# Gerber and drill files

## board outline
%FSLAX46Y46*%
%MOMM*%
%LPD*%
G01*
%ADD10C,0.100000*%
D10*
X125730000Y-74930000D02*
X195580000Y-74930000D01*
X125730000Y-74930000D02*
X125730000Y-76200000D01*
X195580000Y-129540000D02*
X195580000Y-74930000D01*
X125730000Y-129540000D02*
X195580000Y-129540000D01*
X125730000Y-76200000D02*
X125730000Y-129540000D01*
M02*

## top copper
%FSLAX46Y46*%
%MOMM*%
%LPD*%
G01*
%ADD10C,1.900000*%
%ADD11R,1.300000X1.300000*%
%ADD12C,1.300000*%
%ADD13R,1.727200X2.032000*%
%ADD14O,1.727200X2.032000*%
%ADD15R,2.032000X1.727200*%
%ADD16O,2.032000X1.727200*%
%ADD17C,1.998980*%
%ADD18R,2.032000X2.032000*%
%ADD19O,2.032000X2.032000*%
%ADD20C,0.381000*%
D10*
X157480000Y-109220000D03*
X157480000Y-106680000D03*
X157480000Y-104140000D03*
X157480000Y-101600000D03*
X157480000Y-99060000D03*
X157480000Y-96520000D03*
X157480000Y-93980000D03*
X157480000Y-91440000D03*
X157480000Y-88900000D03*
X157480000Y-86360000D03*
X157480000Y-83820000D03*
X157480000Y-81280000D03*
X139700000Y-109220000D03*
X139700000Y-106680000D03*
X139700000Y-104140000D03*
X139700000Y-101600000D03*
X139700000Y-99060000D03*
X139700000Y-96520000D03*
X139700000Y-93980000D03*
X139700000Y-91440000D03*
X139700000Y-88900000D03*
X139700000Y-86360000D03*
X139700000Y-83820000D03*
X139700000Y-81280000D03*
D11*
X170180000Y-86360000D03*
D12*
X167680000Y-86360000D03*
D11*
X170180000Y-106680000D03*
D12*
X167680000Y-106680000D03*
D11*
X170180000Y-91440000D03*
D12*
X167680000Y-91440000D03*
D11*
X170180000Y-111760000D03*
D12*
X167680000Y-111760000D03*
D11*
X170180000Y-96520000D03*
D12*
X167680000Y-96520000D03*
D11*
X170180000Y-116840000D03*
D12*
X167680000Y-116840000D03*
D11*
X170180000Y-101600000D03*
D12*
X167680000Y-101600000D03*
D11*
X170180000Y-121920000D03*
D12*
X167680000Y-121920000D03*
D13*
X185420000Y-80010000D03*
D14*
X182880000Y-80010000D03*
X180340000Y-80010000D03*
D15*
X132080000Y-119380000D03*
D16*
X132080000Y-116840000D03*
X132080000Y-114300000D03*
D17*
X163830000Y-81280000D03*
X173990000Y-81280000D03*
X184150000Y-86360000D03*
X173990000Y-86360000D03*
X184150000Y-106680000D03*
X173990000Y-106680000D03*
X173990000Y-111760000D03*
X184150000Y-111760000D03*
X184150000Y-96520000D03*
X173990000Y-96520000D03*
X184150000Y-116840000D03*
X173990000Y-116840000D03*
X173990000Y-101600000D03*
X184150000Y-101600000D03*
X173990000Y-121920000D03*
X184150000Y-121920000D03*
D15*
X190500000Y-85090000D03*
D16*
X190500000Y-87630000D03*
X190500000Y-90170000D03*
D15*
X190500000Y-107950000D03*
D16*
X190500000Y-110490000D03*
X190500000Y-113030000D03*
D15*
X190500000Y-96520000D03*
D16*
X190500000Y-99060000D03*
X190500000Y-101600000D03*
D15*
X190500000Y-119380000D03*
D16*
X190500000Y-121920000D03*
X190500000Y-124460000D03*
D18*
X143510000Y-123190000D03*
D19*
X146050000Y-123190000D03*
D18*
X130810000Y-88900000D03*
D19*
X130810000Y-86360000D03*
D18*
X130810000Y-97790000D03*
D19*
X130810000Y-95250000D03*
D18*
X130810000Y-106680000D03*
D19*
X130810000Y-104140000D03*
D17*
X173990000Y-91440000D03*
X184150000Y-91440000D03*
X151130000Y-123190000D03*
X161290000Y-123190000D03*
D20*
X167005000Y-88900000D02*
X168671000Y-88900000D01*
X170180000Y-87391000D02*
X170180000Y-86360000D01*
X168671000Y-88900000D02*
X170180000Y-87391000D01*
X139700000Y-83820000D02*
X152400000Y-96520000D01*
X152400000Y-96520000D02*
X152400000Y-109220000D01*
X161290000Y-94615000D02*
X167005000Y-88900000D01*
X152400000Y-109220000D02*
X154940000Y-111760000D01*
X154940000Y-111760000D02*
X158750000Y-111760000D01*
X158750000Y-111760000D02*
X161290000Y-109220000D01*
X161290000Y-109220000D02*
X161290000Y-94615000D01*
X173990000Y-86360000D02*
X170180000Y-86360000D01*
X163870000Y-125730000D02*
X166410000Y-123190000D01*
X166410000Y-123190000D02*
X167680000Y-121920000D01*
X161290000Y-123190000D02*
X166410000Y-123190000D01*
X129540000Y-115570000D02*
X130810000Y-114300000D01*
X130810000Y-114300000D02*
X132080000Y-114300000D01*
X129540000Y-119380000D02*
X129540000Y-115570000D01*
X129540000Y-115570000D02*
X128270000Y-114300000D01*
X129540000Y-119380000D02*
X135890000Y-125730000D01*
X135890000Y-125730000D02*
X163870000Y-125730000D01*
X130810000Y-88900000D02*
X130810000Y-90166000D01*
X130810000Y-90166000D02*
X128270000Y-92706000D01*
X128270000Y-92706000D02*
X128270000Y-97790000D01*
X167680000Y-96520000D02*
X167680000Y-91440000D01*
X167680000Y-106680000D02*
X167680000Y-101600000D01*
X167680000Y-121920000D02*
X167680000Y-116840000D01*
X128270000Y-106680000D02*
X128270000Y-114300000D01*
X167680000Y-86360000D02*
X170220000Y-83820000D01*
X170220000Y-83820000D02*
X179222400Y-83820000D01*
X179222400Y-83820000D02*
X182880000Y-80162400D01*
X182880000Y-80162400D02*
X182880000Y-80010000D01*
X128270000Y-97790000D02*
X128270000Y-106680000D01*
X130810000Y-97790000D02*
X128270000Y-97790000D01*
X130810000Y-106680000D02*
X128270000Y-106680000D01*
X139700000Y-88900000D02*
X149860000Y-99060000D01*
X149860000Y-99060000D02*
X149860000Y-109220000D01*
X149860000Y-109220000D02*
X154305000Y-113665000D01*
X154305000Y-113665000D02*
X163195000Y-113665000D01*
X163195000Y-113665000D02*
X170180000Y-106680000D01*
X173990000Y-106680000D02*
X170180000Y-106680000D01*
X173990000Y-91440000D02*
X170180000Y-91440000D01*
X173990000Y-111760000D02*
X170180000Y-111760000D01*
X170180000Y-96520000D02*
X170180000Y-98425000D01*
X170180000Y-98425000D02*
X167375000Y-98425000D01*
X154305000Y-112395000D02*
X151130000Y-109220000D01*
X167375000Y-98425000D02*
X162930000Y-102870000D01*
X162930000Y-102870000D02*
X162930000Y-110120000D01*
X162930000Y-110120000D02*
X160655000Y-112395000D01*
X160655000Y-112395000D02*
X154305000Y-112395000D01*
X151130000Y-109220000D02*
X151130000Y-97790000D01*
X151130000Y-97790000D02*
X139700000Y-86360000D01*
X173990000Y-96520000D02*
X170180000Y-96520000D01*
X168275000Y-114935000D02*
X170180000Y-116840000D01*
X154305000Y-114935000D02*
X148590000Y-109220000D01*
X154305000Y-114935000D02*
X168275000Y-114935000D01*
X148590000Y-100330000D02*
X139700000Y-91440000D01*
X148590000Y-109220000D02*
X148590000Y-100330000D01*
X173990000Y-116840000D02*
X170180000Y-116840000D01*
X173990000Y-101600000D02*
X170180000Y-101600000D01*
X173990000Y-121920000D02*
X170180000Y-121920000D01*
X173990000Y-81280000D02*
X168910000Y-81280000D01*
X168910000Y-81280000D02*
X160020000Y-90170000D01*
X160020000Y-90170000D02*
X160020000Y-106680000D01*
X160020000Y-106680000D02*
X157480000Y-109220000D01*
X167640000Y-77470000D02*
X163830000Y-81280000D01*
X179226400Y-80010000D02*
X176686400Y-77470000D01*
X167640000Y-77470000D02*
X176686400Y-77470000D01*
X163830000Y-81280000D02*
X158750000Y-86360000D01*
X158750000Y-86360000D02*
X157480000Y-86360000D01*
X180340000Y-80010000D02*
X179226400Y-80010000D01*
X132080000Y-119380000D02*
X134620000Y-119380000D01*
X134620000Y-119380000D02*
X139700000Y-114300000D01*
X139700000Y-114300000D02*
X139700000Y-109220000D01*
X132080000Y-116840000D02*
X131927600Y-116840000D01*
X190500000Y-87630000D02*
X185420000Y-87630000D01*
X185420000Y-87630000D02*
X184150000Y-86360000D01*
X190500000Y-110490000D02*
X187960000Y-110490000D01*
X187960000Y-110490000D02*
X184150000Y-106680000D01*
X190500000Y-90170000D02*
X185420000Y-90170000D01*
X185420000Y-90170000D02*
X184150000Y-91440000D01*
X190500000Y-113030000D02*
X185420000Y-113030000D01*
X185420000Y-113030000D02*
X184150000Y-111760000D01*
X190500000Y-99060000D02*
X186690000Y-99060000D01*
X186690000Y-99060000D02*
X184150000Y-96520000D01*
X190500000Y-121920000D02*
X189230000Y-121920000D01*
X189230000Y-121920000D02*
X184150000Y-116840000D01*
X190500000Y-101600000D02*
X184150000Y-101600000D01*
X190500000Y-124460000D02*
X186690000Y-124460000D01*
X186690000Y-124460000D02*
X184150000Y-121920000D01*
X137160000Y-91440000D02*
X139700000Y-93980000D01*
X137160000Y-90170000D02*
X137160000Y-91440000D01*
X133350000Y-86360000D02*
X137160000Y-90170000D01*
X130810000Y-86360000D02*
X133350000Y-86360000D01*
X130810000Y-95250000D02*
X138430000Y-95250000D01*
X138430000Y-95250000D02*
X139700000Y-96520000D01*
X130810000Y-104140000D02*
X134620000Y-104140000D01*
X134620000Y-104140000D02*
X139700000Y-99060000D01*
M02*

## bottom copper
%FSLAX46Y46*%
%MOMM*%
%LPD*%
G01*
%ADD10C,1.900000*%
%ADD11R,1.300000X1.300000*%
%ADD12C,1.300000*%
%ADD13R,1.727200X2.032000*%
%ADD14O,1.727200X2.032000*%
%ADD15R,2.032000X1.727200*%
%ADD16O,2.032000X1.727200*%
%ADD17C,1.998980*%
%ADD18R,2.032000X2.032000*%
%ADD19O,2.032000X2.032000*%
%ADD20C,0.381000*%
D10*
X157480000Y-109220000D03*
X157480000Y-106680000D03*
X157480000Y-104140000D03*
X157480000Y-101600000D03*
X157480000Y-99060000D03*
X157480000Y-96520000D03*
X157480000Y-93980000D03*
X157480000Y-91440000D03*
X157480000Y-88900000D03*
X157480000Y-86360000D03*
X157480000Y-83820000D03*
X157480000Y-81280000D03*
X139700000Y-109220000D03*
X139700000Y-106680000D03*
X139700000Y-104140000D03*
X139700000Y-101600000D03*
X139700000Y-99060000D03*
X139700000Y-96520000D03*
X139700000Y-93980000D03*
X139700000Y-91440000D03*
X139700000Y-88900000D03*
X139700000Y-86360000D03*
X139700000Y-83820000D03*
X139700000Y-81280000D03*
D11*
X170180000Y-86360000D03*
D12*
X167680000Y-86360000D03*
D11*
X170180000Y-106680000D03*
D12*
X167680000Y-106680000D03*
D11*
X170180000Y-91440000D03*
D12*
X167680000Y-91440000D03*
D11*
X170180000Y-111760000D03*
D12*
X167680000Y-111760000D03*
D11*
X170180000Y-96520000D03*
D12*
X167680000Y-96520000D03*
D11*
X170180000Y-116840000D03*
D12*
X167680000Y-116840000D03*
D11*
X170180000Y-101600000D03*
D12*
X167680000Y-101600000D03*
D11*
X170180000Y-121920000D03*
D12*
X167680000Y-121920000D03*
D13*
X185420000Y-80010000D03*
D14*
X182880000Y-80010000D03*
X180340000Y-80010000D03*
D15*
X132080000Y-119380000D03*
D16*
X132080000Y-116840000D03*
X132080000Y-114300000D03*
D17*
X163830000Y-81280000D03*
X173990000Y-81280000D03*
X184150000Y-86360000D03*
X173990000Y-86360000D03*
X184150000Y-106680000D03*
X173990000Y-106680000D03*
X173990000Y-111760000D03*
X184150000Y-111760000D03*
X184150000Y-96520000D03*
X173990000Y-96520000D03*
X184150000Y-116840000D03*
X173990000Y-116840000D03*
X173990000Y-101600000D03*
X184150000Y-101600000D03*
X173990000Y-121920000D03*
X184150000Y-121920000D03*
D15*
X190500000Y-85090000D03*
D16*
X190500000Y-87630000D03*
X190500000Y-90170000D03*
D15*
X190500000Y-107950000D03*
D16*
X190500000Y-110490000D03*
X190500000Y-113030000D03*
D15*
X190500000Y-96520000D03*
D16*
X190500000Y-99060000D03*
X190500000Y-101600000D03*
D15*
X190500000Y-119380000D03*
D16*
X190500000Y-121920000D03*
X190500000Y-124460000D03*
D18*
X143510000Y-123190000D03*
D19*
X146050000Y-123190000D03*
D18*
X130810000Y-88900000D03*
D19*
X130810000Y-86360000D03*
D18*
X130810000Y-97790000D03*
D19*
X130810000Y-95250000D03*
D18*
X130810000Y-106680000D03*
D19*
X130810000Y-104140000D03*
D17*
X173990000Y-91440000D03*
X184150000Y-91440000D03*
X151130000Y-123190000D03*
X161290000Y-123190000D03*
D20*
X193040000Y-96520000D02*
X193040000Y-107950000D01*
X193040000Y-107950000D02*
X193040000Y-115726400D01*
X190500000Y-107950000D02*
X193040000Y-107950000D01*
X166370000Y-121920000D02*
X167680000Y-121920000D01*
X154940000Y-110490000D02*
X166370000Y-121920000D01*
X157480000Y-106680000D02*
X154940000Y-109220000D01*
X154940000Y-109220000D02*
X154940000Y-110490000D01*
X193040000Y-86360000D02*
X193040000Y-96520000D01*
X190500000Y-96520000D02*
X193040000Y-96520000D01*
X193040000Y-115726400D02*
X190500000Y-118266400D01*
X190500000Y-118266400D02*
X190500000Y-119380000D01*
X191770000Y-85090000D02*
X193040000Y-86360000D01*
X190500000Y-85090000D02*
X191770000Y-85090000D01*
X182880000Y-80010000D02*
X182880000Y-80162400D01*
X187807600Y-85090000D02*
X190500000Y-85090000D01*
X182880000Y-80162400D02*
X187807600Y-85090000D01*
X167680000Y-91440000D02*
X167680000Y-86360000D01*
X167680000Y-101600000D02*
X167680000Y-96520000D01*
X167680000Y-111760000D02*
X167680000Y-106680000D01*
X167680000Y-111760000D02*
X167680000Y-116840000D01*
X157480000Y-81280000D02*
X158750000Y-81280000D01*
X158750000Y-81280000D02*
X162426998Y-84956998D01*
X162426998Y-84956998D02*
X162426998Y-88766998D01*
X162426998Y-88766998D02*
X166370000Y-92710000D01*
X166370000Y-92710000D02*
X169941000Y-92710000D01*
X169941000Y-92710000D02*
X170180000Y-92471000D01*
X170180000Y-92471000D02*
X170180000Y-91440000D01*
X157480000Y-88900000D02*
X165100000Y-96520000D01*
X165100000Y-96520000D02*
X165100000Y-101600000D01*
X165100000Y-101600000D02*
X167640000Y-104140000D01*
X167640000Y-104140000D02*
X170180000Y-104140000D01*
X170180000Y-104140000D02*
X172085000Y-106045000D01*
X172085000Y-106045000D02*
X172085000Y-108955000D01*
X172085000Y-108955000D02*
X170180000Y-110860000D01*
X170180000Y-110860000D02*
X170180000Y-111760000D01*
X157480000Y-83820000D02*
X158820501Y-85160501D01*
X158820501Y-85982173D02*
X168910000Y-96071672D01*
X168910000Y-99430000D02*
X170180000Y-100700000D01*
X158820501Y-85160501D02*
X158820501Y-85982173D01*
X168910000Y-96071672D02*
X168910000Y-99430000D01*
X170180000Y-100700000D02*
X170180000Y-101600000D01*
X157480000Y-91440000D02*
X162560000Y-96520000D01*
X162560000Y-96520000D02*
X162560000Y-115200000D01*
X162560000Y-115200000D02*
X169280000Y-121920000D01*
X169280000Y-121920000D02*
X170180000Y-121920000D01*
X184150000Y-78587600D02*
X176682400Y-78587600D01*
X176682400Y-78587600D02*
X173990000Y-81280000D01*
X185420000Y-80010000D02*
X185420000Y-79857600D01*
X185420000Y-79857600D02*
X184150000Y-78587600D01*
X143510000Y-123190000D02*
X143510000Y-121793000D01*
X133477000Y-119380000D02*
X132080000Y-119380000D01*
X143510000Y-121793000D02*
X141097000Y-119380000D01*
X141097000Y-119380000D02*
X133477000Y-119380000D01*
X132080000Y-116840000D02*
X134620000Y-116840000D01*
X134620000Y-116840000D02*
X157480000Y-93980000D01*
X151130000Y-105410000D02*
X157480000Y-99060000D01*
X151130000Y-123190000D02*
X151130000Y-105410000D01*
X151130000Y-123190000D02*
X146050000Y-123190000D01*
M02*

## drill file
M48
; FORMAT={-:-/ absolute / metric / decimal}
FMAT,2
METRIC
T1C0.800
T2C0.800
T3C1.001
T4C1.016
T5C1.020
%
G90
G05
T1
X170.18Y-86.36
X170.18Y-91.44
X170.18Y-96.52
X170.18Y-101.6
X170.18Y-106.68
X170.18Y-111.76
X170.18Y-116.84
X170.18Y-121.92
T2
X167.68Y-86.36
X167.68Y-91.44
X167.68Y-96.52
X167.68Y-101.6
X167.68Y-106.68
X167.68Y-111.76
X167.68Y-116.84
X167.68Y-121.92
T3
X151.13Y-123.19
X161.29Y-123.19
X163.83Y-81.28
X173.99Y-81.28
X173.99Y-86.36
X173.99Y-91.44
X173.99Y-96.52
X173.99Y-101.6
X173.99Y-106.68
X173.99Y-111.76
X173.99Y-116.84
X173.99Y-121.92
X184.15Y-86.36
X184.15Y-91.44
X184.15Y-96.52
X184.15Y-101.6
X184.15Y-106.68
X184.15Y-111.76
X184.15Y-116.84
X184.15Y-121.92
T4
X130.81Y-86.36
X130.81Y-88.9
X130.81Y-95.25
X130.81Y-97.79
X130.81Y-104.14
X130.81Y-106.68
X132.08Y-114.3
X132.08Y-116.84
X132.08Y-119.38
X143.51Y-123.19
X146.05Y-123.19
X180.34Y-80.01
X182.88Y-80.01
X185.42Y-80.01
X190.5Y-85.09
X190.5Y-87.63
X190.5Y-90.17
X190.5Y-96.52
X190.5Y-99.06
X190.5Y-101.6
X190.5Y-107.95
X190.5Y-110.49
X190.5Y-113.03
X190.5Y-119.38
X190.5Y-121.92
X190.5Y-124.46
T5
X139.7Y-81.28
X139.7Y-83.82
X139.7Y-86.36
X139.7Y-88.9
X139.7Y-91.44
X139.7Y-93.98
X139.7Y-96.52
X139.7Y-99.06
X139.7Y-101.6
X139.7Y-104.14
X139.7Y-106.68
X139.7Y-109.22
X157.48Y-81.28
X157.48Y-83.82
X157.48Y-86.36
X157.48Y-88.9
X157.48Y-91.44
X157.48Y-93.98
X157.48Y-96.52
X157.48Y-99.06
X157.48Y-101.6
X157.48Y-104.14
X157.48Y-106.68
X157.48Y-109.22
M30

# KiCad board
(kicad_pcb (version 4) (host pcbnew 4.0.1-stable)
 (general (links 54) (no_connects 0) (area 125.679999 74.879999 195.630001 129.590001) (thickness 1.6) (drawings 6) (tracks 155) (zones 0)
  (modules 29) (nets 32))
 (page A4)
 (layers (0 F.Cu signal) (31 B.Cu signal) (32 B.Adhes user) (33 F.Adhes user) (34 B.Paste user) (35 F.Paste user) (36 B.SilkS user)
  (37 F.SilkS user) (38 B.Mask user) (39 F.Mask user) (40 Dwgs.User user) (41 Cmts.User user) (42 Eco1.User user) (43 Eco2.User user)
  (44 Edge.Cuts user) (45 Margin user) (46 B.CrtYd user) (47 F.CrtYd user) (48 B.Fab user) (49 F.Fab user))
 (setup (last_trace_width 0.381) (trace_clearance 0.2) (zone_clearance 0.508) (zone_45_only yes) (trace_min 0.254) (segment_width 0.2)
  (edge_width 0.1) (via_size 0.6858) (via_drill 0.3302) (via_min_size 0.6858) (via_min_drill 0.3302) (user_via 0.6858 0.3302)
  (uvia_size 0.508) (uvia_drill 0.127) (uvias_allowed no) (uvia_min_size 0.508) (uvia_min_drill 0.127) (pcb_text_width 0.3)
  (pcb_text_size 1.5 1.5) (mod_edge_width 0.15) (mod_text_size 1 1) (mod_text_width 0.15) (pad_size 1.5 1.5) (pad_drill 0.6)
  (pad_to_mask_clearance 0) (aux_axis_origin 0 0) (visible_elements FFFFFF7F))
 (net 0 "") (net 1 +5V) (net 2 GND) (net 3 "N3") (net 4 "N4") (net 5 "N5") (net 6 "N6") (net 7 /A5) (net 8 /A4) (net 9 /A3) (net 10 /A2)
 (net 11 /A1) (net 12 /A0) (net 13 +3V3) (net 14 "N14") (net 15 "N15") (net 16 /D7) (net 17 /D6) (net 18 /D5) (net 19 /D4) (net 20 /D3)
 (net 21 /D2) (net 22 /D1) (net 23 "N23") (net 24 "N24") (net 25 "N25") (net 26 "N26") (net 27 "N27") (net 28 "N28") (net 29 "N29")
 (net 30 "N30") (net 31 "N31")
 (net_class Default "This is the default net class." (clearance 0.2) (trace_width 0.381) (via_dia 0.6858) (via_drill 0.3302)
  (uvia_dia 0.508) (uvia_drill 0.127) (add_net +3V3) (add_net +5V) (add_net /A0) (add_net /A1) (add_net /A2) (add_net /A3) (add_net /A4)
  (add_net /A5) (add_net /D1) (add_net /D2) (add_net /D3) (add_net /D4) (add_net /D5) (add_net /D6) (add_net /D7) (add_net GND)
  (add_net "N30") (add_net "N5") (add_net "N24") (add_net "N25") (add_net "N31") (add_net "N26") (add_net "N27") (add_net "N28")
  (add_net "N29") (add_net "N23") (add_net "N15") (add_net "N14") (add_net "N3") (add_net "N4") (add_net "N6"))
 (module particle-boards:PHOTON (layer F.Cu) (at 148.59 93.98 180)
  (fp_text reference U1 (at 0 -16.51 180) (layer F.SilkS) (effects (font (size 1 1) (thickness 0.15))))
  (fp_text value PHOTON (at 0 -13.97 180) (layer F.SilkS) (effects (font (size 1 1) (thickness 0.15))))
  (pad 1 thru_hole circle (at -8.89 -15.24 180) (size 1.9 1.9) (drill 1.02) (layers *.Cu *.Mask F.SilkS) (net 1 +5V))
  (pad 2 thru_hole circle (at -8.89 -12.7 180) (size 1.9 1.9) (drill 1.02) (layers *.Cu *.Mask F.SilkS) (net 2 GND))
  (pad 3 thru_hole circle (at -8.89 -10.16 180) (size 1.9 1.9) (drill 1.02) (layers *.Cu *.Mask F.SilkS) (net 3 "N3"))
  (pad 4 thru_hole circle (at -8.89 -7.62 180) (size 1.9 1.9) (drill 1.02) (layers *.Cu *.Mask F.SilkS) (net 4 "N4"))
  (pad 5 thru_hole circle (at -8.89 -5.08 180) (size 1.9 1.9) (drill 1.02) (layers *.Cu *.Mask F.SilkS) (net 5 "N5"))
  (pad 6 thru_hole circle (at -8.89 -2.54 180) (size 1.9 1.9) (drill 1.02) (layers *.Cu *.Mask F.SilkS) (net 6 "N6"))
  (pad 7 thru_hole circle (at -8.89 0 180) (size 1.9 1.9) (drill 1.02) (layers *.Cu *.Mask F.SilkS) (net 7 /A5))
  (pad 8 thru_hole circle (at -8.89 2.54 180) (size 1.9 1.9) (drill 1.02) (layers *.Cu *.Mask F.SilkS) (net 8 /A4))
  (pad 9 thru_hole circle (at -8.89 5.08 180) (size 1.9 1.9) (drill 1.02) (layers *.Cu *.Mask F.SilkS) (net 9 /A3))
  (pad 10 thru_hole circle (at -8.89 7.62 180) (size 1.9 1.9) (drill 1.02) (layers *.Cu *.Mask F.SilkS) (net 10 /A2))
  (pad 11 thru_hole circle (at -8.89 10.16 180) (size 1.9 1.9) (drill 1.02) (layers *.Cu *.Mask F.SilkS) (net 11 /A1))
  (pad 12 thru_hole circle (at -8.89 12.7 180) (size 1.9 1.9) (drill 1.02) (layers *.Cu *.Mask F.SilkS) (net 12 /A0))
  (pad 24 thru_hole circle (at 8.89 -15.24 180) (size 1.9 1.9) (drill 1.02) (layers *.Cu *.Mask F.SilkS) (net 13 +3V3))
  (pad 23 thru_hole circle (at 8.89 -12.7 180) (size 1.9 1.9) (drill 1.02) (layers *.Cu *.Mask F.SilkS) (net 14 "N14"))
  (pad 22 thru_hole circle (at 8.89 -10.16 180) (size 1.9 1.9) (drill 1.02) (layers *.Cu *.Mask F.SilkS) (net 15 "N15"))
  (pad 21 thru_hole circle (at 8.89 -7.62 180) (size 1.9 1.9) (drill 1.02) (layers *.Cu *.Mask F.SilkS))
  (pad 20 thru_hole circle (at 8.89 -5.08 180) (size 1.9 1.9) (drill 1.02) (layers *.Cu *.Mask F.SilkS) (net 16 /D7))
  (pad 19 thru_hole circle (at 8.89 -2.54 180) (size 1.9 1.9) (drill 1.02) (layers *.Cu *.Mask F.SilkS) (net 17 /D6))
  (pad 18 thru_hole circle (at 8.89 0 180) (size 1.9 1.9) (drill 1.02) (layers *.Cu *.Mask F.SilkS) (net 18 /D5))
  (pad 17 thru_hole circle (at 8.89 2.54 180) (size 1.9 1.9) (drill 1.02) (layers *.Cu *.Mask F.SilkS) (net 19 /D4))
  (pad 16 thru_hole circle (at 8.89 5.08 180) (size 1.9 1.9) (drill 1.02) (layers *.Cu *.Mask F.SilkS) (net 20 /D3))
  (pad 15 thru_hole circle (at 8.89 7.62 180) (size 1.9 1.9) (drill 1.02) (layers *.Cu *.Mask F.SilkS) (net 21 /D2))
  (pad 14 thru_hole circle (at 8.89 10.16 180) (size 1.9 1.9) (drill 1.02) (layers *.Cu *.Mask F.SilkS) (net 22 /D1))
  (pad 13 thru_hole circle (at 8.89 12.7 180) (size 1.9 1.9) (drill 1.02) (layers *.Cu *.Mask F.SilkS) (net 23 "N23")))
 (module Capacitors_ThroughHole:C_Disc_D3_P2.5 (layer F.Cu) (at 170.18 86.36 180)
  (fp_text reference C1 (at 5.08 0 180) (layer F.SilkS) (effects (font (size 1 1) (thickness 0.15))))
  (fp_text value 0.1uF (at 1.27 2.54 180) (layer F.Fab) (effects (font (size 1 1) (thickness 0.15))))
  (pad 1 thru_hole rect (at 0 0 180) (size 1.3 1.3) (drill 0.8) (layers *.Cu *.Mask F.SilkS) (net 22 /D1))
  (pad 2 thru_hole circle (at 2.5 0 180) (size 1.3 1.3) (drill 0.8001) (layers *.Cu *.Mask F.SilkS) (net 2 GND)))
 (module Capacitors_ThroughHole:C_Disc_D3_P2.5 (layer F.Cu) (at 170.18 106.68 180)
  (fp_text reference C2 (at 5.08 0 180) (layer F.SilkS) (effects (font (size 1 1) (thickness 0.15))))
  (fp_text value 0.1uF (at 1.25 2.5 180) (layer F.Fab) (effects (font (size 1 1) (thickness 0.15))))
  (pad 1 thru_hole rect (at 0 0 180) (size 1.3 1.3) (drill 0.8) (layers *.Cu *.Mask F.SilkS) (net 20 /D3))
  (pad 2 thru_hole circle (at 2.5 0 180) (size 1.3 1.3) (drill 0.8001) (layers *.Cu *.Mask F.SilkS) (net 2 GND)))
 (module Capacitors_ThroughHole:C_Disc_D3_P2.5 (layer F.Cu) (at 170.18 91.44 180)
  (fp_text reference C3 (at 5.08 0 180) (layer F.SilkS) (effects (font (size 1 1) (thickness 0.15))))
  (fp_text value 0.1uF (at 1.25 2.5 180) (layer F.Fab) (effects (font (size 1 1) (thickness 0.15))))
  (pad 1 thru_hole rect (at 0 0 180) (size 1.3 1.3) (drill 0.8) (layers *.Cu *.Mask F.SilkS) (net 12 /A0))
  (pad 2 thru_hole circle (at 2.5 0 180) (size 1.3 1.3) (drill 0.8001) (layers *.Cu *.Mask F.SilkS) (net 2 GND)))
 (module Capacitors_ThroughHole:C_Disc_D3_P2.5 (layer F.Cu) (at 170.18 111.76 180)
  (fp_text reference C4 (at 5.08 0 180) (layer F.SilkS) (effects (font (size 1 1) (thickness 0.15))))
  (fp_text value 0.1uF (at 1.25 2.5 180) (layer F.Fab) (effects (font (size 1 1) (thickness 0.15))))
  (pad 1 thru_hole rect (at 0 0 180) (size 1.3 1.3) (drill 0.8) (layers *.Cu *.Mask F.SilkS) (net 9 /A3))
  (pad 2 thru_hole circle (at 2.5 0 180) (size 1.3 1.3) (drill 0.8001) (layers *.Cu *.Mask F.SilkS) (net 2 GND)))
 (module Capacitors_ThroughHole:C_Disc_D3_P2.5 (layer F.Cu) (at 170.18 96.52 180)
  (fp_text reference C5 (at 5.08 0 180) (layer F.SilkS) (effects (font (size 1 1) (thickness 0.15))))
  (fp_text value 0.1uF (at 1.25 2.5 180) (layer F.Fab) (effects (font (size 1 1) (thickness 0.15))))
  (pad 1 thru_hole rect (at 0 0 180) (size 1.3 1.3) (drill 0.8) (layers *.Cu *.Mask F.SilkS) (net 21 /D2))
  (pad 2 thru_hole circle (at 2.5 0 180) (size 1.3 1.3) (drill 0.8001) (layers *.Cu *.Mask F.SilkS) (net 2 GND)))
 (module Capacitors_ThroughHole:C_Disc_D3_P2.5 (layer F.Cu) (at 170.18 116.84 180)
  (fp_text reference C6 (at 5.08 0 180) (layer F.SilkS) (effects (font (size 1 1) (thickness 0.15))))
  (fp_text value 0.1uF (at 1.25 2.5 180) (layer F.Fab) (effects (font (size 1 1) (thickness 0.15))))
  (pad 1 thru_hole rect (at 0 0 180) (size 1.3 1.3) (drill 0.8) (layers *.Cu *.Mask F.SilkS) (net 19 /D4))
  (pad 2 thru_hole circle (at 2.5 0 180) (size 1.3 1.3) (drill 0.8001) (layers *.Cu *.Mask F.SilkS) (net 2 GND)))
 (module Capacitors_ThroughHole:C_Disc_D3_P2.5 (layer F.Cu) (at 170.18 101.6 180)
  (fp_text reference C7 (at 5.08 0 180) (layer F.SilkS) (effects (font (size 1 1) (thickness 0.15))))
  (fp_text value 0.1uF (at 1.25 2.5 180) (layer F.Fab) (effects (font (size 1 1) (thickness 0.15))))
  (pad 1 thru_hole rect (at 0 0 180) (size 1.3 1.3) (drill 0.8) (layers *.Cu *.Mask F.SilkS) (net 11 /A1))
  (pad 2 thru_hole circle (at 2.5 0 180) (size 1.3 1.3) (drill 0.8001) (layers *.Cu *.Mask F.SilkS) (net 2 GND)))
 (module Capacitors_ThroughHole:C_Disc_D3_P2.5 (layer F.Cu) (at 170.18 121.92 180)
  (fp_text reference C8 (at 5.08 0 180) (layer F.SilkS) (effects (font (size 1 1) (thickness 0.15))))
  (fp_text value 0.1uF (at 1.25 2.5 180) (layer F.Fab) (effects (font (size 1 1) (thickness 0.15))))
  (pad 1 thru_hole rect (at 0 0 180) (size 1.3 1.3) (drill 0.8) (layers *.Cu *.Mask F.SilkS) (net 8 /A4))
  (pad 2 thru_hole circle (at 2.5 0 180) (size 1.3 1.3) (drill 0.8001) (layers *.Cu *.Mask F.SilkS) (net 2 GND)))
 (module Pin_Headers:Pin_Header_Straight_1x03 (layer F.Cu) (at 185.42 80.01 270)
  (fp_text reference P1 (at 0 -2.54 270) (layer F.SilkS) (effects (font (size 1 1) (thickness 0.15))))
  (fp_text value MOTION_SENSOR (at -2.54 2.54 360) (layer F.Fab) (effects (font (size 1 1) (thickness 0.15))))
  (pad 1 thru_hole rect (at 0 0 270) (size 2.032 1.7272) (drill 1.016) (layers *.Cu *.Mask F.SilkS) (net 1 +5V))
  (pad 2 thru_hole oval (at 0 2.54 270) (size 2.032 1.7272) (drill 1.016) (layers *.Cu *.Mask F.SilkS) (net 2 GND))
  (pad 3 thru_hole oval (at 0 5.08 270) (size 2.032 1.7272) (drill 1.016) (layers *.Cu *.Mask F.SilkS) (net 10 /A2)))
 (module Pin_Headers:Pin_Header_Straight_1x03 (layer F.Cu) (at 132.08 119.38 180)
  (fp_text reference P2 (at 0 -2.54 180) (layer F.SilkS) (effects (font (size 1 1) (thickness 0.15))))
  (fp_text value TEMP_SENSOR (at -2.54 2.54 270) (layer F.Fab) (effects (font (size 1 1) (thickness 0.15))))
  (pad 1 thru_hole rect (at 0 0 180) (size 2.032 1.7272) (drill 1.016) (layers *.Cu *.Mask F.SilkS) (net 13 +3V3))
  (pad 2 thru_hole oval (at 0 2.54 180) (size 2.032 1.7272) (drill 1.016) (layers *.Cu *.Mask F.SilkS) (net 7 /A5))
  (pad 3 thru_hole oval (at 0 5.08 180) (size 2.032 1.7272) (drill 1.016) (layers *.Cu *.Mask F.SilkS) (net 2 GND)))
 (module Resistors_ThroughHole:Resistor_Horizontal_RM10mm (layer F.Cu) (at 168.91 81.28)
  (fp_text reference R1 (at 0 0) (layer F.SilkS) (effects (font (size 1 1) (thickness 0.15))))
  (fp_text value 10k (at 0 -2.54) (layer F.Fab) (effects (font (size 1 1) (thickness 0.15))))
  (pad 1 thru_hole circle (at -5.08 0) (size 1.99898 1.99898) (drill 1.00076) (layers *.Cu *.SilkS *.Mask) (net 10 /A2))
  (pad 2 thru_hole circle (at 5.08 0) (size 1.99898 1.99898) (drill 1.00076) (layers *.Cu *.SilkS *.Mask) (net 1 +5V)))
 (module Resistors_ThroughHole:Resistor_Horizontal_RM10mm (layer F.Cu) (at 179.07 86.36 180)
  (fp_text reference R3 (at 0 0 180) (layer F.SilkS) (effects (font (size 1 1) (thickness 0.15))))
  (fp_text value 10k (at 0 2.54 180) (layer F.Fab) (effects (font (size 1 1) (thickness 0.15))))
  (pad 1 thru_hole circle (at -5.08 0 180) (size 1.99898 1.99898) (drill 1.00076) (layers *.Cu *.SilkS *.Mask) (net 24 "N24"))
  (pad 2 thru_hole circle (at 5.08 0 180) (size 1.99898 1.99898) (drill 1.00076) (layers *.Cu *.SilkS *.Mask) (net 22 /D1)))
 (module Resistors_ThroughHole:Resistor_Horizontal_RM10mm (layer F.Cu) (at 179.07 106.68 180)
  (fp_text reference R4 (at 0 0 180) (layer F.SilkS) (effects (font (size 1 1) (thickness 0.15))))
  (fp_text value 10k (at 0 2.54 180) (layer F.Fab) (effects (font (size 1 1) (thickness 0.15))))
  (pad 1 thru_hole circle (at -5.08 0 180) (size 1.99898 1.99898) (drill 1.00076) (layers *.Cu *.SilkS *.Mask) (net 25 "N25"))
  (pad 2 thru_hole circle (at 5.08 0 180) (size 1.99898 1.99898) (drill 1.00076) (layers *.Cu *.SilkS *.Mask) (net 20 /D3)))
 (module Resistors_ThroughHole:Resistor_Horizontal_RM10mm (layer F.Cu) (at 179.07 111.76)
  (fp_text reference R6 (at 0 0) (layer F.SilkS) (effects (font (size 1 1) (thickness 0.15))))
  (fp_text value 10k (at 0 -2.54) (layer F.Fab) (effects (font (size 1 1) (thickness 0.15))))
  (pad 1 thru_hole circle (at -5.08 0) (size 1.99898 1.99898) (drill 1.00076) (layers *.Cu *.SilkS *.Mask) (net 9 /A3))
  (pad 2 thru_hole circle (at 5.08 0) (size 1.99898 1.99898) (drill 1.00076) (layers *.Cu *.SilkS *.Mask) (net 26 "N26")))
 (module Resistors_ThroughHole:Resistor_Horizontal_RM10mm (layer F.Cu) (at 179.07 96.52 180)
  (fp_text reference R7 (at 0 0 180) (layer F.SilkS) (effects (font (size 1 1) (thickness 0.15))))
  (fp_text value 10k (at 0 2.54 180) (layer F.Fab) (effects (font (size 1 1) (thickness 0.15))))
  (pad 1 thru_hole circle (at -5.08 0 180) (size 1.99898 1.99898) (drill 1.00076) (layers *.Cu *.SilkS *.Mask) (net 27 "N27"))
  (pad 2 thru_hole circle (at 5.08 0 180) (size 1.99898 1.99898) (drill 1.00076) (layers *.Cu *.SilkS *.Mask) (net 21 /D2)))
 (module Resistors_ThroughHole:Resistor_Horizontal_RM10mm (layer F.Cu) (at 179.07 116.84 180)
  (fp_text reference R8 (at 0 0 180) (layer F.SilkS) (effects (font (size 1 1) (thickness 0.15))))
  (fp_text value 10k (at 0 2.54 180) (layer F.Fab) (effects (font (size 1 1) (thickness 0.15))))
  (pad 1 thru_hole circle (at -5.08 0 180) (size 1.99898 1.99898) (drill 1.00076) (layers *.Cu *.SilkS *.Mask) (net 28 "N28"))
  (pad 2 thru_hole circle (at 5.08 0 180) (size 1.99898 1.99898) (drill 1.00076) (layers *.Cu *.SilkS *.Mask) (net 19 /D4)))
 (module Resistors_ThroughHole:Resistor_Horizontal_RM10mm (layer F.Cu) (at 179.07 101.6)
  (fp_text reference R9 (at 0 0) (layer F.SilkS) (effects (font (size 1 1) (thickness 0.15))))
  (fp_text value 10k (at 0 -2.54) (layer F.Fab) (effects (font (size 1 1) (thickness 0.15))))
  (pad 1 thru_hole circle (at -5.08 0) (size 1.99898 1.99898) (drill 1.00076) (layers *.Cu *.SilkS *.Mask) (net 11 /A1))
  (pad 2 thru_hole circle (at 5.08 0) (size 1.99898 1.99898) (drill 1.00076) (layers *.Cu *.SilkS *.Mask) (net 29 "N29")))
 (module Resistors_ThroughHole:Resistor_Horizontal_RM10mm (layer F.Cu) (at 179.07 121.92)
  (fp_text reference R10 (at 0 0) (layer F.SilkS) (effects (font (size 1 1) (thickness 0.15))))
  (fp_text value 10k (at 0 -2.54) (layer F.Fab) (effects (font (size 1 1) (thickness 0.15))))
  (pad 1 thru_hole circle (at -5.08 0) (size 1.99898 1.99898) (drill 1.00076) (layers *.Cu *.SilkS *.Mask) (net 8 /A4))
  (pad 2 thru_hole circle (at 5.08 0) (size 1.99898 1.99898) (drill 1.00076) (layers *.Cu *.SilkS *.Mask) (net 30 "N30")))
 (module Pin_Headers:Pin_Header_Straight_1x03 (layer F.Cu) (at 190.5 85.09)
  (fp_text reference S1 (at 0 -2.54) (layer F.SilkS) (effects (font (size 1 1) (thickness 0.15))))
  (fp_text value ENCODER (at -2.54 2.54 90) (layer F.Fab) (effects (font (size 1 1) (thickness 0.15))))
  (pad 1 thru_hole rect (at 0 0) (size 2.032 1.7272) (drill 1.016) (layers *.Cu *.Mask F.SilkS) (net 2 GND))
  (pad 2 thru_hole oval (at 0 2.54) (size 2.032 1.7272) (drill 1.016) (layers *.Cu *.Mask F.SilkS) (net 24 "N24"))
  (pad 3 thru_hole oval (at 0 5.08) (size 2.032 1.7272) (drill 1.016) (layers *.Cu *.Mask F.SilkS) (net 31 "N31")))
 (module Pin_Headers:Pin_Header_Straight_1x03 (layer F.Cu) (at 190.5 107.95)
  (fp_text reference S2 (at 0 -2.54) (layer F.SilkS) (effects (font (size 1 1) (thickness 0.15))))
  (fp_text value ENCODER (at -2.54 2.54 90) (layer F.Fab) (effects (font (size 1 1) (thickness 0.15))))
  (pad 1 thru_hole rect (at 0 0) (size 2.032 1.7272) (drill 1.016) (layers *.Cu *.Mask F.SilkS) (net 2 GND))
  (pad 2 thru_hole oval (at 0 2.54) (size 2.032 1.7272) (drill 1.016) (layers *.Cu *.Mask F.SilkS) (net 25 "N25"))
  (pad 3 thru_hole oval (at 0 5.08) (size 2.032 1.7272) (drill 1.016) (layers *.Cu *.Mask F.SilkS) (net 26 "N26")))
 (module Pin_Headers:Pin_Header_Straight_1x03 (layer F.Cu) (at 190.5 96.52)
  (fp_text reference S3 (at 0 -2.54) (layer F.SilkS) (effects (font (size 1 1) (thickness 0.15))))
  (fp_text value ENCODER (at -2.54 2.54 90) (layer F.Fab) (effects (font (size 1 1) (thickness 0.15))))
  (pad 1 thru_hole rect (at 0 0) (size 2.032 1.7272) (drill 1.016) (layers *.Cu *.Mask F.SilkS) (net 2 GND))
  (pad 2 thru_hole oval (at 0 2.54) (size 2.032 1.7272) (drill 1.016) (layers *.Cu *.Mask F.SilkS) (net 27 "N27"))
  (pad 3 thru_hole oval (at 0 5.08) (size 2.032 1.7272) (drill 1.016) (layers *.Cu *.Mask F.SilkS) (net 29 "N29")))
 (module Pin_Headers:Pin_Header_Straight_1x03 (layer F.Cu) (at 190.5 119.38)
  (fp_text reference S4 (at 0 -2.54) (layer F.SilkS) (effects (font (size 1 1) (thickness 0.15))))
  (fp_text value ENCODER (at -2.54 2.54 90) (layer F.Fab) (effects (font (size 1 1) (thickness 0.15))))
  (pad 1 thru_hole rect (at 0 0) (size 2.032 1.7272) (drill 1.016) (layers *.Cu *.Mask F.SilkS) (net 2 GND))
  (pad 2 thru_hole oval (at 0 2.54) (size 2.032 1.7272) (drill 1.016) (layers *.Cu *.Mask F.SilkS) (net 28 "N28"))
  (pad 3 thru_hole oval (at 0 5.08) (size 2.032 1.7272) (drill 1.016) (layers *.Cu *.Mask F.SilkS) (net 30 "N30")))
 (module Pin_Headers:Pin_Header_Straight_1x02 (layer F.Cu) (at 143.51 123.19 90)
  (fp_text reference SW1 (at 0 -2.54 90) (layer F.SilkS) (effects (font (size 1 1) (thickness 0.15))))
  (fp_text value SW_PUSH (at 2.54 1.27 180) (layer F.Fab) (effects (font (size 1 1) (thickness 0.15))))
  (pad 1 thru_hole rect (at 0 0 90) (size 2.032 2.032) (drill 1.016) (layers *.Cu *.Mask F.SilkS) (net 13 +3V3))
  (pad 2 thru_hole oval (at 0 2.54 90) (size 2.032 2.032) (drill 1.016) (layers *.Cu *.Mask F.SilkS) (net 5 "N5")))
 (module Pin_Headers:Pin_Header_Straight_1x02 (layer F.Cu) (at 130.81 88.9 180)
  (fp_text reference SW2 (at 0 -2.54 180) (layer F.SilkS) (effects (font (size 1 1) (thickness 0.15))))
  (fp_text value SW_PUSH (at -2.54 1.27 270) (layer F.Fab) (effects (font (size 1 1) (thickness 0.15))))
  (pad 1 thru_hole rect (at 0 0 180) (size 2.032 2.032) (drill 1.016) (layers *.Cu *.Mask F.SilkS) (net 2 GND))
  (pad 2 thru_hole oval (at 0 2.54 180) (size 2.032 2.032) (drill 1.016) (layers *.Cu *.Mask F.SilkS) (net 18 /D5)))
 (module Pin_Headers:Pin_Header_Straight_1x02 (layer F.Cu) (at 130.81 97.79 180)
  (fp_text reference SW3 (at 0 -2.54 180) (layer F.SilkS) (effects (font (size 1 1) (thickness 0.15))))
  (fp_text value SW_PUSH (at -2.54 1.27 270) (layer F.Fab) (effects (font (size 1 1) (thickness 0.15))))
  (pad 1 thru_hole rect (at 0 0 180) (size 2.032 2.032) (drill 1.016) (layers *.Cu *.Mask F.SilkS) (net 2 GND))
  (pad 2 thru_hole oval (at 0 2.54 180) (size 2.032 2.032) (drill 1.016) (layers *.Cu *.Mask F.SilkS) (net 17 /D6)))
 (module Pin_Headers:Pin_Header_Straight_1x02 (layer F.Cu) (at 130.81 106.68 180)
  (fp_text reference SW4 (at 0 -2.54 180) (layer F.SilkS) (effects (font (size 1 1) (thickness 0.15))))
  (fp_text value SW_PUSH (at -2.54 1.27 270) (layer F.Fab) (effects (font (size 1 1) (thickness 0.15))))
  (pad 1 thru_hole rect (at 0 0 180) (size 2.032 2.032) (drill 1.016) (layers *.Cu *.Mask F.SilkS) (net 2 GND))
  (pad 2 thru_hole oval (at 0 2.54 180) (size 2.032 2.032) (drill 1.016) (layers *.Cu *.Mask F.SilkS) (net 16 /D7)))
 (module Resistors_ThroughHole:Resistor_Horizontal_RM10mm (layer F.Cu) (at 179.07 91.44)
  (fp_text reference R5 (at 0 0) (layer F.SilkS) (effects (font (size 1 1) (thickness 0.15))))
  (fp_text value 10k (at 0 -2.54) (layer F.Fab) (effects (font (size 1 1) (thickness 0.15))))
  (pad 1 thru_hole circle (at -5.08 0) (size 1.99898 1.99898) (drill 1.00076) (layers *.Cu *.SilkS *.Mask) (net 12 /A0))
  (pad 2 thru_hole circle (at 5.08 0) (size 1.99898 1.99898) (drill 1.00076) (layers *.Cu *.SilkS *.Mask) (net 31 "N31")))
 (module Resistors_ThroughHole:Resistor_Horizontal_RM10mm (layer F.Cu) (at 156.21 123.19)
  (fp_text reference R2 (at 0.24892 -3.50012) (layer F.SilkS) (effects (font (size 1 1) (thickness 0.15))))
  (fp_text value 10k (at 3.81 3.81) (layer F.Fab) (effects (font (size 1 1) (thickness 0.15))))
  (pad 1 thru_hole circle (at -5.08 0) (size 1.99898 1.99898) (drill 1.00076) (layers *.Cu *.SilkS *.Mask) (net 5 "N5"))
  (pad 2 thru_hole circle (at 5.08 0) (size 1.99898 1.99898) (drill 1.00076) (layers *.Cu *.SilkS *.Mask) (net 2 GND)))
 (gr_line (start 125.73 74.93) (end 195.58 74.93) (layer Edge.Cuts) (width 0.1))
 (gr_line (start 125.73 74.93) (end 125.73 76.2) (layer Edge.Cuts) (width 0.1))
 (gr_line (start 195.58 129.54) (end 195.58 74.93) (layer Edge.Cuts) (width 0.1))
 (gr_line (start 125.73 129.54) (end 195.58 129.54) (layer Edge.Cuts) (width 0.1))
 (gr_line (start 125.73 76.2) (end 125.73 129.54) (layer Edge.Cuts) (width 0.1))
 (segment (start 167.005 88.9) (end 168.671 88.9) (width 0.381) (layer F.Cu) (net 22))
 (segment (start 170.18 87.391) (end 170.18 86.36) (width 0.381) (layer F.Cu) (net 22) (status 20))
 (segment (start 168.671 88.9) (end 170.18 87.391) (width 0.381) (layer F.Cu) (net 22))
 (segment (start 139.7 83.82) (end 152.4 96.52) (width 0.381) (layer F.Cu) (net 22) (status 10))
 (segment (start 152.4 96.52) (end 152.4 109.22) (width 0.381) (layer F.Cu) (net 22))
 (segment (start 161.29 94.615) (end 167.005 88.9) (width 0.381) (layer F.Cu) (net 22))
 (segment (start 152.4 109.22) (end 154.94 111.76) (width 0.381) (layer F.Cu) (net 22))
 (segment (start 154.94 111.76) (end 158.75 111.76) (width 0.381) (layer F.Cu) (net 22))
 (segment (start 158.75 111.76) (end 161.29 109.22) (width 0.381) (layer F.Cu) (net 22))
 (segment (start 161.29 109.22) (end 161.29 94.615) (width 0.381) (layer F.Cu) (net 22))
 (segment (start 173.99 86.36) (end 170.18 86.36) (width 0.381) (layer F.Cu) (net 22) (status 30))
 (segment (start 163.87 125.73) (end 166.41 123.19) (width 0.381) (layer F.Cu) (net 2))
 (segment (start 166.41 123.19) (end 167.68 121.92) (width 0.381) (layer F.Cu) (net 2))
 (segment (start 161.29 123.19) (end 166.41 123.19) (width 0.381) (layer F.Cu) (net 2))
 (segment (start 193.04 96.52) (end 193.04 107.95) (width 0.381) (layer B.Cu) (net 2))
 (segment (start 193.04 107.95) (end 193.04 115.7264) (width 0.381) (layer B.Cu) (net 2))
 (segment (start 190.5 107.95) (end 193.04 107.95) (width 0.381) (layer B.Cu) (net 2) (status 10))
 (segment (start 166.37 121.92) (end 167.68 121.92) (width 0.381) (layer B.Cu) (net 2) (status 20))
 (segment (start 154.94 110.49) (end 166.37 121.92) (width 0.381) (layer B.Cu) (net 2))
 (segment (start 157.48 106.68) (end 154.94 109.22) (width 0.381) (layer B.Cu) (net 2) (status 10))
 (segment (start 154.94 109.22) (end 154.94 110.49) (width 0.381) (layer B.Cu) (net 2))
 (segment (start 129.54 115.57) (end 130.81 114.3) (width 0.381) (layer F.Cu) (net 2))
 (segment (start 130.81 114.3) (end 132.08 114.3) (width 0.381) (layer F.Cu) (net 2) (status 20))
 (segment (start 129.54 119.38) (end 129.54 115.57) (width 0.381) (layer F.Cu) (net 2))
 (segment (start 129.54 115.57) (end 128.27 114.3) (width 0.381) (layer F.Cu) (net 2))
 (segment (start 129.54 119.38) (end 135.89 125.73) (width 0.381) (layer F.Cu) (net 2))
 (segment (start 135.89 125.73) (end 163.87 125.73) (width 0.381) (layer F.Cu) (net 2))
 (segment (start 130.81 88.9) (end 130.81 90.166) (width 0.381) (layer F.Cu) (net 2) (status 10))
 (segment (start 130.81 90.166) (end 128.27 92.706) (width 0.381) (layer F.Cu) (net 2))
 (segment (start 128.27 92.706) (end 128.27 97.79) (width 0.381) (layer F.Cu) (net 2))
 (segment (start 167.68 96.52) (end 167.68 91.44) (width 0.381) (layer F.Cu) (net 2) (status 30))
 (segment (start 167.68 106.68) (end 167.68 101.6) (width 0.381) (layer F.Cu) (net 2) (status 30))
 (segment (start 167.68 121.92) (end 167.68 116.84) (width 0.381) (layer F.Cu) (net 2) (status 30))
 (segment (start 128.27 106.68) (end 128.27 114.3) (width 0.381) (layer F.Cu) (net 2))
 (segment (start 167.68 86.36) (end 170.22 83.82) (width 0.381) (layer F.Cu) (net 2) (status 10))
 (segment (start 170.22 83.82) (end 179.2224 83.82) (width 0.381) (layer F.Cu) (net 2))
 (segment (start 179.2224 83.82) (end 182.88 80.1624) (width 0.381) (layer F.Cu) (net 2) (status 20))
 (segment (start 182.88 80.1624) (end 182.88 80.01) (width 0.381) (layer F.Cu) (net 2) (status 30))
 (segment (start 128.27 97.79) (end 128.27 106.68) (width 0.381) (layer F.Cu) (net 2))
 (segment (start 130.81 97.79) (end 128.27 97.79) (width 0.381) (layer F.Cu) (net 2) (status 10))
 (segment (start 130.81 106.68) (end 128.27 106.68) (width 0.381) (layer F.Cu) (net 2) (status 10))
 (segment (start 193.04 86.36) (end 193.04 96.52) (width 0.381) (layer B.Cu) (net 2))
 (segment (start 190.5 96.52) (end 193.04 96.52) (width 0.381) (layer B.Cu) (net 2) (status 10))
 (segment (start 193.04 115.7264) (end 190.5 118.2664) (width 0.381) (layer B.Cu) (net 2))
 (segment (start 190.5 118.2664) (end 190.5 119.38) (width 0.381) (layer B.Cu) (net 2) (status 20))
 (segment (start 191.77 85.09) (end 193.04 86.36) (width 0.381) (layer B.Cu) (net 2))
 (segment (start 190.5 85.09) (end 191.77 85.09) (width 0.381) (layer B.Cu) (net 2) (status 10))
 (segment (start 182.88 80.01) (end 182.88 80.1624) (width 0.381) (layer B.Cu) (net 2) (status 30))
 (segment (start 187.8076 85.09) (end 190.5 85.09) (width 0.381) (layer B.Cu) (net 2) (status 20))
 (segment (start 182.88 80.1624) (end 187.8076 85.09) (width 0.381) (layer B.Cu) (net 2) (status 10))
 (segment (start 167.68 91.44) (end 167.68 86.36) (width 0.381) (layer B.Cu) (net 2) (status 30))
 (segment (start 167.68 101.6) (end 167.68 96.52) (width 0.381) (layer B.Cu) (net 2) (status 30))
 (segment (start 167.68 111.76) (end 167.68 106.68) (width 0.381) (layer B.Cu) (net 2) (status 30))
 (segment (start 167.68 111.76) (end 167.68 116.84) (width 0.381) (layer B.Cu) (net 2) (status 30))
 (segment (start 139.7 88.9) (end 149.86 99.06) (width 0.381) (layer F.Cu) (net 20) (status 10))
 (segment (start 149.86 99.06) (end 149.86 109.22) (width 0.381) (layer F.Cu) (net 20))
 (segment (start 149.86 109.22) (end 154.305 113.665) (width 0.381) (layer F.Cu) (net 20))
 (segment (start 154.305 113.665) (end 163.195 113.665) (width 0.381) (layer F.Cu) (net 20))
 (segment (start 163.195 113.665) (end 170.18 106.68) (width 0.381) (layer F.Cu) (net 20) (status 20))
 (segment (start 173.99 106.68) (end 170.18 106.68) (width 0.381) (layer F.Cu) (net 20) (status 30))
 (segment (start 157.48 81.28) (end 158.75 81.28) (width 0.381) (layer B.Cu) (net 12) (status 10))
 (segment (start 158.75 81.28) (end 162.426998 84.956998) (width 0.381) (layer B.Cu) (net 12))
 (segment (start 162.426998 84.956998) (end 162.426998 88.766998) (width 0.381) (layer B.Cu) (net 12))
 (segment (start 162.426998 88.766998) (end 166.37 92.71) (width 0.381) (layer B.Cu) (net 12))
 (segment (start 166.37 92.71) (end 169.941 92.71) (width 0.381) (layer B.Cu) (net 12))
 (segment (start 169.941 92.71) (end 170.18 92.471) (width 0.381) (layer B.Cu) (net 12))
 (segment (start 170.18 92.471) (end 170.18 91.44) (width 0.381) (layer B.Cu) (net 12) (status 20))
 (segment (start 173.99 91.44) (end 170.18 91.44) (width 0.381) (layer F.Cu) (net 12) (status 30))
 (segment (start 157.48 88.9) (end 165.1 96.52) (width 0.381) (layer B.Cu) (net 9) (status 10))
 (segment (start 165.1 96.52) (end 165.1 101.6) (width 0.381) (layer B.Cu) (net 9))
 (segment (start 165.1 101.6) (end 167.64 104.14) (width 0.381) (layer B.Cu) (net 9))
 (segment (start 167.64 104.14) (end 170.18 104.14) (width 0.381) (layer B.Cu) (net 9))
 (segment (start 170.18 104.14) (end 172.085 106.045) (width 0.381) (layer B.Cu) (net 9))
 (segment (start 172.085 106.045) (end 172.085 108.955) (width 0.381) (layer B.Cu) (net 9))
 (segment (start 172.085 108.955) (end 170.18 110.86) (width 0.381) (layer B.Cu) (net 9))
 (segment (start 170.18 110.86) (end 170.18 111.76) (width 0.381) (layer B.Cu) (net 9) (status 20))
 (segment (start 173.99 111.76) (end 170.18 111.76) (width 0.381) (layer F.Cu) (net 9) (status 30))
 (segment (start 170.18 96.52) (end 170.18 98.425) (width 0.381) (layer F.Cu) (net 21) (status 10))
 (segment (start 170.18 98.425) (end 167.375 98.425) (width 0.381) (layer F.Cu) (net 21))
 (segment (start 154.305 112.395) (end 151.13 109.22) (width 0.381) (layer F.Cu) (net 21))
 (segment (start 167.375 98.425) (end 162.93 102.87) (width 0.381) (layer F.Cu) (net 21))
 (segment (start 162.93 102.87) (end 162.93 110.12) (width 0.381) (layer F.Cu) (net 21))
 (segment (start 162.93 110.12) (end 160.655 112.395) (width 0.381) (layer F.Cu) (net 21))
 (segment (start 160.655 112.395) (end 154.305 112.395) (width 0.381) (layer F.Cu) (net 21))
 (segment (start 151.13 109.22) (end 151.13 97.79) (width 0.381) (layer F.Cu) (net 21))
 (segment (start 151.13 97.79) (end 139.7 86.36) (width 0.381) (layer F.Cu) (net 21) (status 20))
 (segment (start 173.99 96.52) (end 170.18 96.52) (width 0.381) (layer F.Cu) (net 21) (status 30))
 (segment (start 168.275 114.935) (end 170.18 116.84) (width 0.381) (layer F.Cu) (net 19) (status 20))
 (segment (start 154.305 114.935) (end 148.59 109.22) (width 0.381) (layer F.Cu) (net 19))
 (segment (start 154.305 114.935) (end 168.275 114.935) (width 0.381) (layer F.Cu) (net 19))
 (segment (start 148.59 100.33) (end 139.7 91.44) (width 0.381) (layer F.Cu) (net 19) (status 20))
 (segment (start 148.59 109.22) (end 148.59 100.33) (width 0.381) (layer F.Cu) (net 19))
 (segment (start 173.99 116.84) (end 170.18 116.84) (width 0.381) (layer F.Cu) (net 19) (status 30))
 (segment (start 157.48 83.82) (end 158.820501 85.160501) (width 0.381) (layer B.Cu) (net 11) (status 10))
 (segment (start 158.820501 85.982173) (end 168.91 96.071672) (width 0.381) (layer B.Cu) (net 11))
 (segment (start 168.91 99.43) (end 170.18 100.7) (width 0.381) (layer B.Cu) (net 11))
 (segment (start 158.820501 85.160501) (end 158.820501 85.982173) (width 0.381) (layer B.Cu) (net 11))
 (segment (start 168.91 96.071672) (end 168.91 99.43) (width 0.381) (layer B.Cu) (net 11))
 (segment (start 170.18 100.7) (end 170.18 101.6) (width 0.381) (layer B.Cu) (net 11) (status 20))
 (segment (start 173.99 101.6) (end 170.18 101.6) (width 0.381) (layer F.Cu) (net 11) (status 30))
 (segment (start 157.48 91.44) (end 162.56 96.52) (width 0.381) (layer B.Cu) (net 8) (status 10))
 (segment (start 162.56 96.52) (end 162.56 115.2) (width 0.381) (layer B.Cu) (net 8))
 (segment (start 162.56 115.2) (end 169.28 121.92) (width 0.381) (layer B.Cu) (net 8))
 (segment (start 169.28 121.92) (end 170.18 121.92) (width 0.381) (layer B.Cu) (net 8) (status 20))
 (segment (start 173.99 121.92) (end 170.18 121.92) (width 0.381) (layer F.Cu) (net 8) (status 30))
 (segment (start 173.99 81.28) (end 168.91 81.28) (width 0.381) (layer F.Cu) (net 1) (status 10))
 (segment (start 168.91 81.28) (end 160.02 90.17) (width 0.381) (layer F.Cu) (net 1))
 (segment (start 160.02 90.17) (end 160.02 106.68) (width 0.381) (layer F.Cu) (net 1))
 (segment (start 160.02 106.68) (end 157.48 109.22) (width 0.381) (layer F.Cu) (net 1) (status 20))
 (segment (start 184.15 78.5876) (end 176.6824 78.5876) (width 0.381) (layer B.Cu) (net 1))
 (segment (start 176.6824 78.5876) (end 173.99 81.28) (width 0.381) (layer B.Cu) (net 1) (status 20))
 (segment (start 185.42 80.01) (end 185.42 79.8576) (width 0.381) (layer B.Cu) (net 1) (status 30))
 (segment (start 185.42 79.8576) (end 184.15 78.5876) (width 0.381) (layer B.Cu) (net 1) (status 10))
 (segment (start 167.64 77.47) (end 163.83 81.28) (width 0.381) (layer F.Cu) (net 10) (status 20))
 (segment (start 179.2264 80.01) (end 176.6864 77.47) (width 0.381) (layer F.Cu) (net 10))
 (segment (start 167.64 77.47) (end 176.6864 77.47) (width 0.381) (layer F.Cu) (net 10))
 (segment (start 163.83 81.28) (end 158.75 86.36) (width 0.381) (layer F.Cu) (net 10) (status 10))
 (segment (start 158.75 86.36) (end 157.48 86.36) (width 0.381) (layer F.Cu) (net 10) (status 20))
 (segment (start 180.34 80.01) (end 179.2264 80.01) (width 0.381) (layer F.Cu) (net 10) (status 10))
 (segment (start 143.51 123.19) (end 143.51 121.793) (width 0.381) (layer B.Cu) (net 13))
 (segment (start 133.477 119.38) (end 132.08 119.38) (width 0.381) (layer B.Cu) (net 13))
 (segment (start 143.51 121.793) (end 141.097 119.38) (width 0.381) (layer B.Cu) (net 13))
 (segment (start 141.097 119.38) (end 133.477 119.38) (width 0.381) (layer B.Cu) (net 13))
 (segment (start 132.08 119.38) (end 134.62 119.38) (width 0.381) (layer F.Cu) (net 13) (status 10))
 (segment (start 134.62 119.38) (end 139.7 114.3) (width 0.381) (layer F.Cu) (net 13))
 (segment (start 139.7 114.3) (end 139.7 109.22) (width 0.381) (layer F.Cu) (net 13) (status 20))
 (segment (start 132.08 116.84) (end 134.62 116.84) (width 0.381) (layer B.Cu) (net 7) (status 10))
 (segment (start 134.62 116.84) (end 157.48 93.98) (width 0.381) (layer B.Cu) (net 7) (status 20))
 (segment (start 132.08 116.84) (end 131.9276 116.84) (width 0.381) (layer F.Cu) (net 7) (status 30))
 (segment (start 190.5 87.63) (end 185.42 87.63) (width 0.381) (layer F.Cu) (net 24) (status 10))
 (segment (start 185.42 87.63) (end 184.15 86.36) (width 0.381) (layer F.Cu) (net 24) (status 20))
 (segment (start 190.5 110.49) (end 187.96 110.49) (width 0.381) (layer F.Cu) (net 25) (status 10))
 (segment (start 187.96 110.49) (end 184.15 106.68) (width 0.381) (layer F.Cu) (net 25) (status 20))
 (segment (start 190.5 90.17) (end 185.42 90.17) (width 0.381) (layer F.Cu) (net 31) (status 10))
 (segment (start 185.42 90.17) (end 184.15 91.44) (width 0.381) (layer F.Cu) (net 31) (status 20))
 (segment (start 190.5 113.03) (end 185.42 113.03) (width 0.381) (layer F.Cu) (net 26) (status 10))
 (segment (start 185.42 113.03) (end 184.15 111.76) (width 0.381) (layer F.Cu) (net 26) (status 20))
 (segment (start 190.5 99.06) (end 186.69 99.06) (width 0.381) (layer F.Cu) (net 27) (status 10))
 (segment (start 186.69 99.06) (end 184.15 96.52) (width 0.381) (layer F.Cu) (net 27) (status 20))
 (segment (start 190.5 121.92) (end 189.23 121.92) (width 0.381) (layer F.Cu) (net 28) (status 10))
 (segment (start 189.23 121.92) (end 184.15 116.84) (width 0.381) (layer F.Cu) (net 28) (status 20))
 (segment (start 190.5 101.6) (end 184.15 101.6) (width 0.381) (layer F.Cu) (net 29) (status 30))
 (segment (start 190.5 124.46) (end 186.69 124.46) (width 0.381) (layer F.Cu) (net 30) (status 10))
 (segment (start 186.69 124.46) (end 184.15 121.92) (width 0.381) (layer F.Cu) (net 30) (status 20))
 (segment (start 151.13 105.41) (end 157.48 99.06) (width 0.381) (layer B.Cu) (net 5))
 (segment (start 151.13 123.19) (end 151.13 105.41) (width 0.381) (layer B.Cu) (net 5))
 (segment (start 151.13 123.19) (end 146.05 123.19) (width 0.381) (layer B.Cu) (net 5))
 (segment (start 137.16 91.44) (end 139.7 93.98) (width 0.381) (layer F.Cu) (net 18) (status 20))
 (segment (start 137.16 90.17) (end 137.16 91.44) (width 0.381) (layer F.Cu) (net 18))
 (segment (start 133.35 86.36) (end 137.16 90.17) (width 0.381) (layer F.Cu) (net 18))
 (segment (start 130.81 86.36) (end 133.35 86.36) (width 0.381) (layer F.Cu) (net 18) (status 10))
 (segment (start 130.81 95.25) (end 138.43 95.25) (width 0.381) (layer F.Cu) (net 17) (status 10))
 (segment (start 138.43 95.25) (end 139.7 96.52) (width 0.381) (layer F.Cu) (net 17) (status 20))
 (segment (start 130.81 104.14) (end 134.62 104.14) (width 0.381) (layer F.Cu) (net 16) (status 10))
 (segment (start 134.62 104.14) (end 139.7 99.06) (width 0.381) (layer F.Cu) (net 16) (status 20)))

